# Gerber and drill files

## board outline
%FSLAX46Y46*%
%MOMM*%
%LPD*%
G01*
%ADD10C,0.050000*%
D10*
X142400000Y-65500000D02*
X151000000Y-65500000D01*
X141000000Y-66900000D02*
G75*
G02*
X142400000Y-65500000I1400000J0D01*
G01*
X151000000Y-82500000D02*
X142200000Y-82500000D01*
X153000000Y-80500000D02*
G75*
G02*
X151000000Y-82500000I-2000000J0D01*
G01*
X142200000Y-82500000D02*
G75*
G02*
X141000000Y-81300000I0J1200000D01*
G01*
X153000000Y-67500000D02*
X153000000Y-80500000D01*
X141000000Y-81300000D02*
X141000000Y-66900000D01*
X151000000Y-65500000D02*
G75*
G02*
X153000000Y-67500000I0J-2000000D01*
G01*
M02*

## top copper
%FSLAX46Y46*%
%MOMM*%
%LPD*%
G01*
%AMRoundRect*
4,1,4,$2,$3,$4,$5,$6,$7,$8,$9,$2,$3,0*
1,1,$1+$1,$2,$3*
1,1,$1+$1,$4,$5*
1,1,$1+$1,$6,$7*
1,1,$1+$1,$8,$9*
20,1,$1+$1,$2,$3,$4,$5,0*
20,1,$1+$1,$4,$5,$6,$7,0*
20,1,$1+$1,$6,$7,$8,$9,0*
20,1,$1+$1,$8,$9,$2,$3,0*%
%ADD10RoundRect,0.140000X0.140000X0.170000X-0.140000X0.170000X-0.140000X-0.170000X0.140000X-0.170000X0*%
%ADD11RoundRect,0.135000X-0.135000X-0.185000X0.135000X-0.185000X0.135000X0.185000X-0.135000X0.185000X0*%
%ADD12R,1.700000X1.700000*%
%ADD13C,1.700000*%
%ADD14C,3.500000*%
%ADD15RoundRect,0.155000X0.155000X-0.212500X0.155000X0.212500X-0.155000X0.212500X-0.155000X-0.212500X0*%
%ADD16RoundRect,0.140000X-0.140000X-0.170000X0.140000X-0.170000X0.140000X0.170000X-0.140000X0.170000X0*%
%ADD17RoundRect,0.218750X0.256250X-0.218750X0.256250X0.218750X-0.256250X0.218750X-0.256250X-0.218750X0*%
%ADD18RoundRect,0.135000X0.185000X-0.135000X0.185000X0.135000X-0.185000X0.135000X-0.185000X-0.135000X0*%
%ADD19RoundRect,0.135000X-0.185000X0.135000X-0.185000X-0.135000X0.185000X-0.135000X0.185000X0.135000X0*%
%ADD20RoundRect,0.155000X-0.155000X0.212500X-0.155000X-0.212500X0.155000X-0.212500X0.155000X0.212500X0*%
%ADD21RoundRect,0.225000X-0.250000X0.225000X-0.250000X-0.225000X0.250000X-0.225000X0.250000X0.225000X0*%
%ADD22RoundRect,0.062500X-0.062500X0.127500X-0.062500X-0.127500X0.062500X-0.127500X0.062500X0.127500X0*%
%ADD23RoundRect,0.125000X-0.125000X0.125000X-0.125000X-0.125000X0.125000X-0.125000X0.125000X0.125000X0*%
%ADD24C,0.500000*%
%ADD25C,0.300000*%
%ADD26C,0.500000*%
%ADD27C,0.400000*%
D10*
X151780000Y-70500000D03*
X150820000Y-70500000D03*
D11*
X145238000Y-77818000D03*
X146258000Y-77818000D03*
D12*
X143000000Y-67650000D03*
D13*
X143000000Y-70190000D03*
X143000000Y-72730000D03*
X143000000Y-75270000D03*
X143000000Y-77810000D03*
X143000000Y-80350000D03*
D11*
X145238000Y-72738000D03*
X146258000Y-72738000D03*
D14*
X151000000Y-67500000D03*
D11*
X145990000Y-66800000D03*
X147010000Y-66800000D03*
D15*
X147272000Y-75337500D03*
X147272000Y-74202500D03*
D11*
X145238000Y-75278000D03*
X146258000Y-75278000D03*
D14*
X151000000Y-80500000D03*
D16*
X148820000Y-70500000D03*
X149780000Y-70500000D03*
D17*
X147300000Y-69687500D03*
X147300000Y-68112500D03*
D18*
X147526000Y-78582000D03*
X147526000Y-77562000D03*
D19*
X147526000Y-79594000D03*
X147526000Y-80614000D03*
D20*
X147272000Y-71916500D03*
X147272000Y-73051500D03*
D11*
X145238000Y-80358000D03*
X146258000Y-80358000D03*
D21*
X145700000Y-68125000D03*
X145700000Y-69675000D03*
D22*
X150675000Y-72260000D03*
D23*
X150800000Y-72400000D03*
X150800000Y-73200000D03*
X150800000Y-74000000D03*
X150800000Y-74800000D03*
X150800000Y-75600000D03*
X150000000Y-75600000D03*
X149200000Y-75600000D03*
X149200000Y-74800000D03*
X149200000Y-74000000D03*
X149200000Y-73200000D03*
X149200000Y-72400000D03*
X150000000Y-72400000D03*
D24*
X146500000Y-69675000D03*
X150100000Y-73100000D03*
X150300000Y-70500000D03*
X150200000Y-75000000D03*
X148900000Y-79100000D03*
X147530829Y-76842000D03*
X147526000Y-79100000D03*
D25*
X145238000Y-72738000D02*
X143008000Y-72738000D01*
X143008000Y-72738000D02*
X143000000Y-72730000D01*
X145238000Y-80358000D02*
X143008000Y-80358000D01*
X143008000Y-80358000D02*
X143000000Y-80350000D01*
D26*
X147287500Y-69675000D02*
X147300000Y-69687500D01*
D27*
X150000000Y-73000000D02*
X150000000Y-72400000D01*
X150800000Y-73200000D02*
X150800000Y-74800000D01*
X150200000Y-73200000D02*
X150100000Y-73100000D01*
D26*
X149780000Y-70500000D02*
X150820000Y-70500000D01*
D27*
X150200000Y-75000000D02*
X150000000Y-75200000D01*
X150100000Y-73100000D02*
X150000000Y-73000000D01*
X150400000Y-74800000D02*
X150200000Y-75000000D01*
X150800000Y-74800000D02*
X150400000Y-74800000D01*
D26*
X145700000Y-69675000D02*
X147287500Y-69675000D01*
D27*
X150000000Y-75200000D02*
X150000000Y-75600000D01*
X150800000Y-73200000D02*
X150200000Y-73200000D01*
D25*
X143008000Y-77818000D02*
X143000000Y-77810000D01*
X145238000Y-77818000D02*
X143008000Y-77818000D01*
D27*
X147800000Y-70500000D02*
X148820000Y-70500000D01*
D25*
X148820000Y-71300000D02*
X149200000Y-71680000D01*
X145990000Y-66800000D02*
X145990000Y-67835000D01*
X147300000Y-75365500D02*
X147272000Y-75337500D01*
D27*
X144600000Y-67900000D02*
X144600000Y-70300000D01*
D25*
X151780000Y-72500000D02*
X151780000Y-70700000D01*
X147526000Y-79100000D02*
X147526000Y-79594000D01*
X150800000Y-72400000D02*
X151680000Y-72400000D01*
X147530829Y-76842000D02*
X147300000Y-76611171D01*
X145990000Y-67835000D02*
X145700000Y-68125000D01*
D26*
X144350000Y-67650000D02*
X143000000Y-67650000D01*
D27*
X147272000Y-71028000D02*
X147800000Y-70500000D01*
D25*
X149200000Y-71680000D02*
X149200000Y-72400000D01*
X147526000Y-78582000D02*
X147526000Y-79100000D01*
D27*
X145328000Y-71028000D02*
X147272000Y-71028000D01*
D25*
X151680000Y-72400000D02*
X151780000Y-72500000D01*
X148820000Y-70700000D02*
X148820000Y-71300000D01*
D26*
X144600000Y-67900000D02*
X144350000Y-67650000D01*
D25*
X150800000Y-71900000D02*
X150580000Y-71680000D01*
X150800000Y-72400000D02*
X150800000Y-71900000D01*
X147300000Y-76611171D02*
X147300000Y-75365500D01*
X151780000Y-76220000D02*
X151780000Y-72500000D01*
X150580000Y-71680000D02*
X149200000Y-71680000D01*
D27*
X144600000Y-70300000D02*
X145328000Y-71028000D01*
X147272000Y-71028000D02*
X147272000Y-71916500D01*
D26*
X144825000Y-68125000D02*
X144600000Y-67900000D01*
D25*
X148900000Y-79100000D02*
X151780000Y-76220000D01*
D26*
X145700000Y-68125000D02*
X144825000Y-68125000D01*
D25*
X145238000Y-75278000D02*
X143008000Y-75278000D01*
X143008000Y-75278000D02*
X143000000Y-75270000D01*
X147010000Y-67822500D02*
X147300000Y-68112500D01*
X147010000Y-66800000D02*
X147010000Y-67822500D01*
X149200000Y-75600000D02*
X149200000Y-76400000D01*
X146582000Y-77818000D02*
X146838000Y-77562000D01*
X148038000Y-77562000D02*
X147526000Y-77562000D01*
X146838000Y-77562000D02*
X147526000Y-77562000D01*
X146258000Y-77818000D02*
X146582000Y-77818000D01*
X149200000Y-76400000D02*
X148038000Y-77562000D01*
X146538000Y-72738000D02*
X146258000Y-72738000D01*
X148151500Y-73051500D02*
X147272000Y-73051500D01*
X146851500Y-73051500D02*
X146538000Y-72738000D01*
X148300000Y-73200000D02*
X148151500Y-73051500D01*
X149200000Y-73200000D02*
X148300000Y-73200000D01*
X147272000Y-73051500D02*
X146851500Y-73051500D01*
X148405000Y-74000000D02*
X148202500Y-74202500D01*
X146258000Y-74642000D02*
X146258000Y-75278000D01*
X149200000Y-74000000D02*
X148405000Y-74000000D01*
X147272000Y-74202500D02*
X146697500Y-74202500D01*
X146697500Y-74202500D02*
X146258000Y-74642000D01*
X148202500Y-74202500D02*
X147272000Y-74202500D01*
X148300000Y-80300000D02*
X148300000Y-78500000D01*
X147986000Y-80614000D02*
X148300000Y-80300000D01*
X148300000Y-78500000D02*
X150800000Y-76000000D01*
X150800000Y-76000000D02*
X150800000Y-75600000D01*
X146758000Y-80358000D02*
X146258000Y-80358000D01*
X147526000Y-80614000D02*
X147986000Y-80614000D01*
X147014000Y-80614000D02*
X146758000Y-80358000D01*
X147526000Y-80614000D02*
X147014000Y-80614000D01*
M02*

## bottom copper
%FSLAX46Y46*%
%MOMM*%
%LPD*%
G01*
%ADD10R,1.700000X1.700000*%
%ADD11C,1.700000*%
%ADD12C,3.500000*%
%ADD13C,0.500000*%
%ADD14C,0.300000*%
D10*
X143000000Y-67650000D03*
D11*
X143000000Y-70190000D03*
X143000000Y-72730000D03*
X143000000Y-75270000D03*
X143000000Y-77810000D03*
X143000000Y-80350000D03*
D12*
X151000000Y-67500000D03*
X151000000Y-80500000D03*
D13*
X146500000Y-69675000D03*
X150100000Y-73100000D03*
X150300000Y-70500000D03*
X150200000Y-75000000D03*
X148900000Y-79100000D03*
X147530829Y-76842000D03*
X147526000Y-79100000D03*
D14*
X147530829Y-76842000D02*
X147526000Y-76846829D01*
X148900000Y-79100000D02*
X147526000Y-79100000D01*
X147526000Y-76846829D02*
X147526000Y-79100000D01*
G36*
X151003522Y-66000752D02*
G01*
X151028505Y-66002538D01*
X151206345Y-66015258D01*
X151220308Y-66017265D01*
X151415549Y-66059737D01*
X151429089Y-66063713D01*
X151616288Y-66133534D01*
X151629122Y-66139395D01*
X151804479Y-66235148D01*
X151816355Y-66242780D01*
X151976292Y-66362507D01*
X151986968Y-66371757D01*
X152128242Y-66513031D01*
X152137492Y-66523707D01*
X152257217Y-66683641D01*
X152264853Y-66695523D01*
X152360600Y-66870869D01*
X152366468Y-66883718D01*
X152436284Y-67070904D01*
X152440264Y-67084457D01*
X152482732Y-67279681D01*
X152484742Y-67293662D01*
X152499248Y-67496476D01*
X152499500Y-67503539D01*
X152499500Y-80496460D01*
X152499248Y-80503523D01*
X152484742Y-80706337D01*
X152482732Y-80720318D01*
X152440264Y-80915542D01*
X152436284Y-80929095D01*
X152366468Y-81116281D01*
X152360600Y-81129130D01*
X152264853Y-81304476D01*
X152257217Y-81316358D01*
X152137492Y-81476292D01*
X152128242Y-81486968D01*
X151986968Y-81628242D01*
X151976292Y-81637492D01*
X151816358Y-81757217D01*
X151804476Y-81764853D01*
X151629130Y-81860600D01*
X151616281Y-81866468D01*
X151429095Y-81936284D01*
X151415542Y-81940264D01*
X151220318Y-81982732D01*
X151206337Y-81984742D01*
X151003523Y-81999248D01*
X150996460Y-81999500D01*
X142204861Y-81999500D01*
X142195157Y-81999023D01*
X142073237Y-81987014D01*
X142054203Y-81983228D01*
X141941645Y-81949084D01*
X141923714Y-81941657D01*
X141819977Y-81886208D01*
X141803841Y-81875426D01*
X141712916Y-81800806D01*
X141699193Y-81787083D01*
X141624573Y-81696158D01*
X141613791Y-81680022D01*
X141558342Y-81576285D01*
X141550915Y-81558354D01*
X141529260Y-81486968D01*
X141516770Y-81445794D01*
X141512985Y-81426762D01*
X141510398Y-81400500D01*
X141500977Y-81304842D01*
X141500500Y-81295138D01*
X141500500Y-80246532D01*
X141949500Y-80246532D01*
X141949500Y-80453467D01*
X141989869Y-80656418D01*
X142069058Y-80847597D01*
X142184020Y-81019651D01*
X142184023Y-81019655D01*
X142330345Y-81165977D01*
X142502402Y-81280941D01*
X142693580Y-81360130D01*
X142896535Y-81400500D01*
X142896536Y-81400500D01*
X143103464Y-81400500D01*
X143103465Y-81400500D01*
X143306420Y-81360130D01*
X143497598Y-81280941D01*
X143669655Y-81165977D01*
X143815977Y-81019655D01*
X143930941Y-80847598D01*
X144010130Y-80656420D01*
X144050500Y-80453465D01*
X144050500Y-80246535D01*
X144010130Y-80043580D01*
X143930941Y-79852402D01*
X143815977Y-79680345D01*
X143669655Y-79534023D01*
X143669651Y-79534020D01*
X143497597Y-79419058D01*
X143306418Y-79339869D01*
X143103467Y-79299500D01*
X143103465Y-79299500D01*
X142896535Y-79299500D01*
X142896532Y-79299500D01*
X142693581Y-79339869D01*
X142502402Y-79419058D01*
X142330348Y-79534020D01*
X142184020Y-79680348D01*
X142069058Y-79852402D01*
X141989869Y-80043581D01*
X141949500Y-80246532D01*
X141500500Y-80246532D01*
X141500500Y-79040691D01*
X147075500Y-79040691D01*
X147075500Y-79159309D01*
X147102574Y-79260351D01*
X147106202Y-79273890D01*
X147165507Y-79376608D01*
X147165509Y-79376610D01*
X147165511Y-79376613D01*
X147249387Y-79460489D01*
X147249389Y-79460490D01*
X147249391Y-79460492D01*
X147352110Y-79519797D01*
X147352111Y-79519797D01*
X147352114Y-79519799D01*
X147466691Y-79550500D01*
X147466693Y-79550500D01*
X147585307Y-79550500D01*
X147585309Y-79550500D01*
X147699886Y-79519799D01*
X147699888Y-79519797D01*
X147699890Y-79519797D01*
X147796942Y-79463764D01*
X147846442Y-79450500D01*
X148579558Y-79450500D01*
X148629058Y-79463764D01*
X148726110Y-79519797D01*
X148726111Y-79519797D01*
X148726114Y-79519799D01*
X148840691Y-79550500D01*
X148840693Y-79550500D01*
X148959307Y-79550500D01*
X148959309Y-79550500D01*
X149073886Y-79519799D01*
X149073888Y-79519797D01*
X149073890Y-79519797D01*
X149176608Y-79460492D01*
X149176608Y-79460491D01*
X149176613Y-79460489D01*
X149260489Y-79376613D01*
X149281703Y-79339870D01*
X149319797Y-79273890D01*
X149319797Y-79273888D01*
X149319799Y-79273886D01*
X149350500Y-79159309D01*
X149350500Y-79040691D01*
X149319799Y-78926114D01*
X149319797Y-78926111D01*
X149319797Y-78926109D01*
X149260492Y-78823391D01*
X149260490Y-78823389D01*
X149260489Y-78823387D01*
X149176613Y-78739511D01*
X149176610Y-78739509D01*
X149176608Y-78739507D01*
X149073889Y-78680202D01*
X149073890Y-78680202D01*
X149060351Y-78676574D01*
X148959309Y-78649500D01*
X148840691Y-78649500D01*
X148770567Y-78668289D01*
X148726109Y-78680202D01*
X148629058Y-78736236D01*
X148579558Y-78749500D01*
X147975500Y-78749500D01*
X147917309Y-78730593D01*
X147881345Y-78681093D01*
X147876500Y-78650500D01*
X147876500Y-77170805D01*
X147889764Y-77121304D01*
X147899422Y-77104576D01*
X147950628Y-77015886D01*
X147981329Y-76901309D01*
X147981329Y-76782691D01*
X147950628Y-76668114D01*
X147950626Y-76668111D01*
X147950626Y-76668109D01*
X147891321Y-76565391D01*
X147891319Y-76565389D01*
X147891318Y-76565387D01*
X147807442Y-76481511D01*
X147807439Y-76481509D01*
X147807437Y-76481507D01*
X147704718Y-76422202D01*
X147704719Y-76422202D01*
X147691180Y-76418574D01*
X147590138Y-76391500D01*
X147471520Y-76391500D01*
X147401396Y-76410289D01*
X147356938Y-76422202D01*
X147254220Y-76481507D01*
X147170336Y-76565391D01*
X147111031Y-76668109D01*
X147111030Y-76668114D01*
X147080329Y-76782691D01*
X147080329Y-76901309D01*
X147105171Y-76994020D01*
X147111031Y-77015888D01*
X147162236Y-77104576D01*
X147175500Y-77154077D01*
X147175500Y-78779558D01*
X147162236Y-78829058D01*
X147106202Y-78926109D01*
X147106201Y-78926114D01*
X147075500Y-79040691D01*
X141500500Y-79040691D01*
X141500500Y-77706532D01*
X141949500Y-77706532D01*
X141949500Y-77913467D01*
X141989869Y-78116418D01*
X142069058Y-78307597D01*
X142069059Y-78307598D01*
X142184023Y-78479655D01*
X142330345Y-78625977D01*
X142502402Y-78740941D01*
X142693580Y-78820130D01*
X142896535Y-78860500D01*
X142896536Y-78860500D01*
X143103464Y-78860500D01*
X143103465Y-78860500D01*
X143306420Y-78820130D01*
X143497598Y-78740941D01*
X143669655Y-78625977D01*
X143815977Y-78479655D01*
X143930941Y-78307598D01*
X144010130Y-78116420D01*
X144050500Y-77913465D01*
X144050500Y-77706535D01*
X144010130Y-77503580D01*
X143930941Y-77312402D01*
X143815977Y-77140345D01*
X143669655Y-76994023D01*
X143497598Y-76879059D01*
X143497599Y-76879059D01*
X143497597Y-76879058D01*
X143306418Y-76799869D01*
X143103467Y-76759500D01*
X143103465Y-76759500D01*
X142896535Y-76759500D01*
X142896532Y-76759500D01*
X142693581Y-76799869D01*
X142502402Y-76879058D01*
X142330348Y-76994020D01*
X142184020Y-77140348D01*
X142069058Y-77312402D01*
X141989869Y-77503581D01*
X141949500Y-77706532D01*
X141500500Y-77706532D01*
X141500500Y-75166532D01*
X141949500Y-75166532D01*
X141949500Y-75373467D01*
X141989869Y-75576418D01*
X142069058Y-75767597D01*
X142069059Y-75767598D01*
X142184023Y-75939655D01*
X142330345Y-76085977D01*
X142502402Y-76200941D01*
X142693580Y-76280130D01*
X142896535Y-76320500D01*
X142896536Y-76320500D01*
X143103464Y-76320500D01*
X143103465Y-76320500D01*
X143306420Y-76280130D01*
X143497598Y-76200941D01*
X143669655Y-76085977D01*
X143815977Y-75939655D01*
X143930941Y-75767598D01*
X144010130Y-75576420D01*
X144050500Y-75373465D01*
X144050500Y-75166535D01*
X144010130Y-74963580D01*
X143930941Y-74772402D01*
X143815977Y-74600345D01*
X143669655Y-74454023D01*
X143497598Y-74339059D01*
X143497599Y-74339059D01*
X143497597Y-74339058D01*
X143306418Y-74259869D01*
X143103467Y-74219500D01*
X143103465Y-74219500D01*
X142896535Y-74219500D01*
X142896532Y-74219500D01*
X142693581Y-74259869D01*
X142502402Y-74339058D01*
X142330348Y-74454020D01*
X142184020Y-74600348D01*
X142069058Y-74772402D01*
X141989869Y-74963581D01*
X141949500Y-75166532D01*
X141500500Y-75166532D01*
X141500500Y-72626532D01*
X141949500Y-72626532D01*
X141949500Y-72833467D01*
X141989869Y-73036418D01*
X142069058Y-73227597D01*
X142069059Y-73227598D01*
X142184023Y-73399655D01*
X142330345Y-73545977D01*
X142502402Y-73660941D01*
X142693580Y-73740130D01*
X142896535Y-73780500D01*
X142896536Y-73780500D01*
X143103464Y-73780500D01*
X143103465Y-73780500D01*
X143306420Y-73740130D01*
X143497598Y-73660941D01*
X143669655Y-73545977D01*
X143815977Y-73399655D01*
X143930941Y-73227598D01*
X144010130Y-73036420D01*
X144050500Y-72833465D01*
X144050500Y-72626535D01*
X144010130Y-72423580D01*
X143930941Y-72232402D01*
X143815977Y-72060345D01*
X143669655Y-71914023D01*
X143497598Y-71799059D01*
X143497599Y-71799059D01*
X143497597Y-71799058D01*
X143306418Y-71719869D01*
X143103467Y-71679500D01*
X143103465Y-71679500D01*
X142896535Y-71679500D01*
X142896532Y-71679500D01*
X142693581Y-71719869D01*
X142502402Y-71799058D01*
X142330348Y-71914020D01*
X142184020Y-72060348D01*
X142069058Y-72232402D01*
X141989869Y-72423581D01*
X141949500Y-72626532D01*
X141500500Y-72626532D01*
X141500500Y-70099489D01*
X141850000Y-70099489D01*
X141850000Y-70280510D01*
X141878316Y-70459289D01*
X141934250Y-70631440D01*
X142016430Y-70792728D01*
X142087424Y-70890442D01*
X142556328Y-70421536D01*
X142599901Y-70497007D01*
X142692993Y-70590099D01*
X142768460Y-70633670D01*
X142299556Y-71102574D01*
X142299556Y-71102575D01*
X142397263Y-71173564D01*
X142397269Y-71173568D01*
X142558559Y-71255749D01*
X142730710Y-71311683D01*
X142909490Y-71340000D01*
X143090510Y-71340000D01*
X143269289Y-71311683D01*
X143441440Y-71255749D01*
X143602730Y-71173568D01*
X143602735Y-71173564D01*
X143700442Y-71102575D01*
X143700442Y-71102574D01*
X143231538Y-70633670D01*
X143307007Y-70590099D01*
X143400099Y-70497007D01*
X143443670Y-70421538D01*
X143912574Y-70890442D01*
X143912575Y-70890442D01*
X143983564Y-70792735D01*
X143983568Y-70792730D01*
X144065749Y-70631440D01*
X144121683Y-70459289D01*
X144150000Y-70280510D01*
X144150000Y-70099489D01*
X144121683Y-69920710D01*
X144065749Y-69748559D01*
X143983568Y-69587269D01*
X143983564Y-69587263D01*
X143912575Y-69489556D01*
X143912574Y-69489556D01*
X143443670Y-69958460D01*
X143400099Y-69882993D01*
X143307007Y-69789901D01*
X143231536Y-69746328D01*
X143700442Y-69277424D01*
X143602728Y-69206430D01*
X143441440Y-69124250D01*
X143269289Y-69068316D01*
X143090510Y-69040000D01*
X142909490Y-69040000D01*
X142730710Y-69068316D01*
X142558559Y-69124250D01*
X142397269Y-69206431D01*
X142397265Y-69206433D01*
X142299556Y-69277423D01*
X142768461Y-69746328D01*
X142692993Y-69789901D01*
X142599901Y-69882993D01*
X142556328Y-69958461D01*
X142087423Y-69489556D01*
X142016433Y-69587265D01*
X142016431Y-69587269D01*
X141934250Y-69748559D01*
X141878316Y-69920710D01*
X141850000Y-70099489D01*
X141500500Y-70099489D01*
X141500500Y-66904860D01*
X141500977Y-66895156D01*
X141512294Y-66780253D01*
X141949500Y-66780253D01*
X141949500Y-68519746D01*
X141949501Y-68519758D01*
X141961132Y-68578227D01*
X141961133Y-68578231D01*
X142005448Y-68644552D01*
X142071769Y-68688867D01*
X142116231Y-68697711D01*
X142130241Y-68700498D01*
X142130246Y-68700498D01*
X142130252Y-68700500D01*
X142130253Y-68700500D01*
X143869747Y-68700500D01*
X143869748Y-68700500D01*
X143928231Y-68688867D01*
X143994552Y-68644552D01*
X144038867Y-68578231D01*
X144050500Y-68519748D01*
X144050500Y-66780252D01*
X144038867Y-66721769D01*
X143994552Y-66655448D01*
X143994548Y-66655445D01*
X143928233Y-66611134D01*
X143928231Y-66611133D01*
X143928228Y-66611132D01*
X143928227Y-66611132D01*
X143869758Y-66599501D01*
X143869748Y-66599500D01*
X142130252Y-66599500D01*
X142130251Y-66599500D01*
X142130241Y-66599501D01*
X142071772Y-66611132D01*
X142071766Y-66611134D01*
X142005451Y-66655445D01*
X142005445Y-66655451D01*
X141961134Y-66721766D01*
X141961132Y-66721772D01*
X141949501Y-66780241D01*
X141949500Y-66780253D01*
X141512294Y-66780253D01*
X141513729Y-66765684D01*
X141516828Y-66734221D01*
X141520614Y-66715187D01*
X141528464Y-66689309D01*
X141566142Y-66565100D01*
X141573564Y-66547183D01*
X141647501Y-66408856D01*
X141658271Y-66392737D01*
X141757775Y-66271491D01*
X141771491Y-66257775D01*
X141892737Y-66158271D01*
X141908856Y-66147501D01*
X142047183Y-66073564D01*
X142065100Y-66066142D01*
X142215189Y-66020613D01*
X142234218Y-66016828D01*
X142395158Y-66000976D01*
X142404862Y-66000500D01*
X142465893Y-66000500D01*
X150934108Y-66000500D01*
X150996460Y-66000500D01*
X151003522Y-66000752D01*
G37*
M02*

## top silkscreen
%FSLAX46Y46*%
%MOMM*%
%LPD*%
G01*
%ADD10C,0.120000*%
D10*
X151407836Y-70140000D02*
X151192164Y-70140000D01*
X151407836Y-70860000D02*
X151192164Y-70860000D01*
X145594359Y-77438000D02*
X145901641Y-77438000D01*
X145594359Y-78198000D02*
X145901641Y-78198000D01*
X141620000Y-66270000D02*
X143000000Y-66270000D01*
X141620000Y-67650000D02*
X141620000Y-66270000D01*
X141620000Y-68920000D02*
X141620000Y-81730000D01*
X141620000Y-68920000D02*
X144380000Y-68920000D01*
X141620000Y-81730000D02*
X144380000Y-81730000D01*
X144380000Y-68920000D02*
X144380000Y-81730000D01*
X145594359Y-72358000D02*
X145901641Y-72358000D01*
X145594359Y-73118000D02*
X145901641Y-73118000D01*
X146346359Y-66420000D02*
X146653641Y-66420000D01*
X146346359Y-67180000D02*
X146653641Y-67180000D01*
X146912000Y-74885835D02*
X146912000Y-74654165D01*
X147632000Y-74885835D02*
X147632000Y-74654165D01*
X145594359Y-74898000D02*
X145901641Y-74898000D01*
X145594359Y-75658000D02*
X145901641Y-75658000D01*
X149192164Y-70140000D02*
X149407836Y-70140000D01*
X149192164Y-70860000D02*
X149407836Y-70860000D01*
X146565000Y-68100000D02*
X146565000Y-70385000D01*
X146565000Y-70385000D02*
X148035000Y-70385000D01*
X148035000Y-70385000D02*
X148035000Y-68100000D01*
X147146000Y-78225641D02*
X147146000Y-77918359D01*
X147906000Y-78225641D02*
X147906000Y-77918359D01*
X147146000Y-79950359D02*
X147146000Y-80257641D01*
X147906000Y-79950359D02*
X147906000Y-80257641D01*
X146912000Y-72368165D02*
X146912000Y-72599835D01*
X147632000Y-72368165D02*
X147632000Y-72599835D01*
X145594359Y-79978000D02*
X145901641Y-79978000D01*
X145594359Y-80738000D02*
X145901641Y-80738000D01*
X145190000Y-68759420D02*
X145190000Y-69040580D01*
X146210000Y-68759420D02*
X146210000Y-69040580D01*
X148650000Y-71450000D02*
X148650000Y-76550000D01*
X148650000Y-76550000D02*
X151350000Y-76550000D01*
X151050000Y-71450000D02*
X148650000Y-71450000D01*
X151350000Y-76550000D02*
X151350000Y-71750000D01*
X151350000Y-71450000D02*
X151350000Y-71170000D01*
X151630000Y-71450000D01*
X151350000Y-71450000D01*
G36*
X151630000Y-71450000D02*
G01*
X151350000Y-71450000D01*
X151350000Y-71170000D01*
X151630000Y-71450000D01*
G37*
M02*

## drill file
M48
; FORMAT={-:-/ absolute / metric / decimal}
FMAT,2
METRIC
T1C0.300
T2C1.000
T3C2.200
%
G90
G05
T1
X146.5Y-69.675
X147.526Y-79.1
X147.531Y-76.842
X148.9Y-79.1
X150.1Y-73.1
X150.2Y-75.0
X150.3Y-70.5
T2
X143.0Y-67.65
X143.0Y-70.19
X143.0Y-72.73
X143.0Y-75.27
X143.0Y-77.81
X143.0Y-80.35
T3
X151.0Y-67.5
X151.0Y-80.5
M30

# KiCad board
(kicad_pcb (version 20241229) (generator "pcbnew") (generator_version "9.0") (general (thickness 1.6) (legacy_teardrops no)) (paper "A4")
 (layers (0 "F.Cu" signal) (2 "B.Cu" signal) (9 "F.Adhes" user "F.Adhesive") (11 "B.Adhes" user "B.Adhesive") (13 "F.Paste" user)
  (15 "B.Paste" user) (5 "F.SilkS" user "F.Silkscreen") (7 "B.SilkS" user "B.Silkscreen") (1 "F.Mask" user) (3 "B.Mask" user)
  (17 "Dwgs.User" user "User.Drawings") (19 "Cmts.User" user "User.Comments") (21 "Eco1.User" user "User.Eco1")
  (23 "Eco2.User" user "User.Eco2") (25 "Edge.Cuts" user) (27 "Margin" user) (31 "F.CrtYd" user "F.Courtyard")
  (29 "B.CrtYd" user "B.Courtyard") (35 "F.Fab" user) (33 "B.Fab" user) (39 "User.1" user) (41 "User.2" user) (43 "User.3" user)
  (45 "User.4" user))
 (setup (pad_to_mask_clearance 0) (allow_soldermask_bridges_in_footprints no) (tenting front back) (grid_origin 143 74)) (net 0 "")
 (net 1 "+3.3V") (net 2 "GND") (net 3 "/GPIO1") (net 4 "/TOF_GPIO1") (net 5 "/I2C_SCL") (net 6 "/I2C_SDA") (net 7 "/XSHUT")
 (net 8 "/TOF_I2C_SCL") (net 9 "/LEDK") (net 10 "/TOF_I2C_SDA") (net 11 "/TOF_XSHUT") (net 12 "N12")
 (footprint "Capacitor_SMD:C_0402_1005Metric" (layer "F.Cu") (at 151.3 70.5 180)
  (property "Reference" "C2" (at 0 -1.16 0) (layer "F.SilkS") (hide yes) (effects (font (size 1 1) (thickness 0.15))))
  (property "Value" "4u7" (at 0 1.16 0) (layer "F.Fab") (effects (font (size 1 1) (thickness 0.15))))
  (fp_line (start -0.107836 0.36) (end 0.107836 0.36) (stroke (width 0.12) (type solid)) (layer "F.SilkS"))
  (fp_line (start -0.107836 -0.36) (end 0.107836 -0.36) (stroke (width 0.12) (type solid)) (layer "F.SilkS"))
  (pad "1" smd roundrect (at -0.48 0 180) (size 0.56 0.62) (layers "F.Cu" "F.Mask" "F.Paste") (roundrect_rratio 0.25) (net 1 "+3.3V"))
  (pad "2" smd roundrect (at 0.48 0 180) (size 0.56 0.62) (layers "F.Cu" "F.Mask" "F.Paste") (roundrect_rratio 0.25) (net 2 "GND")))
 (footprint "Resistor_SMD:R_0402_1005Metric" (layer "F.Cu") (at 145.748 77.818)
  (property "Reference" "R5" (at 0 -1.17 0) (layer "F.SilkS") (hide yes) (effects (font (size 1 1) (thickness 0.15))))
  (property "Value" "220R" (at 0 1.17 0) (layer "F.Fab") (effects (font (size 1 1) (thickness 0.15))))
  (fp_line (start -0.153641 -0.38) (end 0.153641 -0.38) (stroke (width 0.12) (type solid)) (layer "F.SilkS"))
  (fp_line (start -0.153641 0.38) (end 0.153641 0.38) (stroke (width 0.12) (type solid)) (layer "F.SilkS"))
  (pad "1" smd roundrect (at -0.51 0) (size 0.54 0.64) (layers "F.Cu" "F.Mask" "F.Paste") (roundrect_rratio 0.25) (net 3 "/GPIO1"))
  (pad "2" smd roundrect (at 0.51 0) (size 0.54 0.64) (layers "F.Cu" "F.Mask" "F.Paste") (roundrect_rratio 0.25) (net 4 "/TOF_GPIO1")))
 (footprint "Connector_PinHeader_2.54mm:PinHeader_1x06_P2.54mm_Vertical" (layer "F.Cu") (at 143 67.65)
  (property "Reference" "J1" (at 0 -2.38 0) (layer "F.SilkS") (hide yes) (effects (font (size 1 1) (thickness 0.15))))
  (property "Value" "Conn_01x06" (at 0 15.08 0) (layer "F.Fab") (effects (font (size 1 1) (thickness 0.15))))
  (fp_line (start -1.38 -1.38) (end 0 -1.38) (stroke (width 0.12) (type solid)) (layer "F.SilkS"))
  (fp_line (start -1.38 0) (end -1.38 -1.38) (stroke (width 0.12) (type solid)) (layer "F.SilkS"))
  (fp_line (start -1.38 1.27) (end -1.38 14.08) (stroke (width 0.12) (type solid)) (layer "F.SilkS"))
  (fp_line (start -1.38 1.27) (end 1.38 1.27) (stroke (width 0.12) (type solid)) (layer "F.SilkS"))
  (fp_line (start -1.38 14.08) (end 1.38 14.08) (stroke (width 0.12) (type solid)) (layer "F.SilkS"))
  (fp_line (start 1.38 1.27) (end 1.38 14.08) (stroke (width 0.12) (type solid)) (layer "F.SilkS"))
  (pad "1" thru_hole rect (at 0 0) (size 1.7 1.7) (drill 1) (layers "*.Cu" "*.Mask") (remove_unused_layers no) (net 1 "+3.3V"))
  (pad "2" thru_hole circle (at 0 2.54) (size 1.7 1.7) (drill 1) (layers "*.Cu" "*.Mask") (remove_unused_layers no) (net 2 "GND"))
  (pad "3" thru_hole circle (at 0 5.08) (size 1.7 1.7) (drill 1) (layers "*.Cu" "*.Mask") (remove_unused_layers no) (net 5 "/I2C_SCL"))
  (pad "4" thru_hole circle (at 0 7.62) (size 1.7 1.7) (drill 1) (layers "*.Cu" "*.Mask") (remove_unused_layers no) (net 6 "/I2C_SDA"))
  (pad "5" thru_hole circle (at 0 10.16) (size 1.7 1.7) (drill 1) (layers "*.Cu" "*.Mask") (remove_unused_layers no) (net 3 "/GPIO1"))
  (pad "6" thru_hole circle (at 0 12.7) (size 1.7 1.7) (drill 1) (layers "*.Cu" "*.Mask") (remove_unused_layers no) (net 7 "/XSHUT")))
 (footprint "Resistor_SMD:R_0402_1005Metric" (layer "F.Cu") (at 145.748 72.738)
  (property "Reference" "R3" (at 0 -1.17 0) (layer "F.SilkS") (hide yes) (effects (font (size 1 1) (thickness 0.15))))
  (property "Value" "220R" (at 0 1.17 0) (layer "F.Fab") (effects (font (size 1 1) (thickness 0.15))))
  (fp_line (start -0.153641 -0.38) (end 0.153641 -0.38) (stroke (width 0.12) (type solid)) (layer "F.SilkS"))
  (fp_line (start -0.153641 0.38) (end 0.153641 0.38) (stroke (width 0.12) (type solid)) (layer "F.SilkS"))
  (pad "1" smd roundrect (at -0.51 0) (size 0.54 0.64) (layers "F.Cu" "F.Mask" "F.Paste") (roundrect_rratio 0.25) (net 5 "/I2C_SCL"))
  (pad "2" smd roundrect (at 0.51 0) (size 0.54 0.64) (layers "F.Cu" "F.Mask" "F.Paste") (roundrect_rratio 0.25) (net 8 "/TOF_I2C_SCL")))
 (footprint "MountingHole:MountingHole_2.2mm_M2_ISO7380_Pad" (layer "F.Cu") (at 151 67.5)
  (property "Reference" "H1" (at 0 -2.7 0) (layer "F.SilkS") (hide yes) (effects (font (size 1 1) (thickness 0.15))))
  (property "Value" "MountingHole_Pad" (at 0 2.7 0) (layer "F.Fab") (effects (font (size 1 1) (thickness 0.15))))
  (pad "1" thru_hole circle (at 0 0) (size 3.5 3.5) (drill 2.2) (layers "*.Cu" "*.Mask") (remove_unused_layers no) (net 2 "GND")
   (zone_connect 2)))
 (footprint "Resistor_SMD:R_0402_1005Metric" (layer "F.Cu") (at 146.5 66.8)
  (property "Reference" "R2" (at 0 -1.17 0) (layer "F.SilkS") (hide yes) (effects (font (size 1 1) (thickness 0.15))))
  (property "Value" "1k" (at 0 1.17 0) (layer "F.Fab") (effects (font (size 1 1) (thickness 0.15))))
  (fp_line (start -0.153641 -0.38) (end 0.153641 -0.38) (stroke (width 0.12) (type solid)) (layer "F.SilkS"))
  (fp_line (start -0.153641 0.38) (end 0.153641 0.38) (stroke (width 0.12) (type solid)) (layer "F.SilkS"))
  (pad "1" smd roundrect (at -0.51 0) (size 0.54 0.64) (layers "F.Cu" "F.Mask" "F.Paste") (roundrect_rratio 0.25) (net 1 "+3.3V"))
  (pad "2" smd roundrect (at 0.51 0) (size 0.54 0.64) (layers "F.Cu" "F.Mask" "F.Paste") (roundrect_rratio 0.25) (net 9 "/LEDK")))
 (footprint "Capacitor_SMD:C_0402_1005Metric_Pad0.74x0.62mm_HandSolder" (layer "F.Cu") (at 147.272 74.77 90)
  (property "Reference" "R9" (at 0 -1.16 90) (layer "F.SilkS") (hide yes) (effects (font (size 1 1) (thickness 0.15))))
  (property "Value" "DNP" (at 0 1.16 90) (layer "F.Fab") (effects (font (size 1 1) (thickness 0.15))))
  (fp_line (start -0.115835 -0.36) (end 0.115835 -0.36) (stroke (width 0.12) (type solid)) (layer "F.SilkS"))
  (fp_line (start -0.115835 0.36) (end 0.115835 0.36) (stroke (width 0.12) (type solid)) (layer "F.SilkS"))
  (pad "1" smd roundrect (at -0.5675 0 90) (size 0.735 0.62) (layers "F.Cu" "F.Mask" "F.Paste") (roundrect_rratio 0.25) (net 1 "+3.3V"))
  (pad "2" smd roundrect (at 0.5675 0 90) (size 0.735 0.62) (layers "F.Cu" "F.Mask" "F.Paste") (roundrect_rratio 0.25)
   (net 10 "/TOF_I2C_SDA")))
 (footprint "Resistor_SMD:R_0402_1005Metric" (layer "F.Cu") (at 145.748 75.278)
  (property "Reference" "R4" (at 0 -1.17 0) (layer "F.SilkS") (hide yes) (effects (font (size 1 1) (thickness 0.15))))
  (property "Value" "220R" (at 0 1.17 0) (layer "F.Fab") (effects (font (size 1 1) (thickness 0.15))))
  (fp_line (start -0.153641 -0.38) (end 0.153641 -0.38) (stroke (width 0.12) (type solid)) (layer "F.SilkS"))
  (fp_line (start -0.153641 0.38) (end 0.153641 0.38) (stroke (width 0.12) (type solid)) (layer "F.SilkS"))
  (pad "1" smd roundrect (at -0.51 0) (size 0.54 0.64) (layers "F.Cu" "F.Mask" "F.Paste") (roundrect_rratio 0.25) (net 6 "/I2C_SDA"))
  (pad "2" smd roundrect (at 0.51 0) (size 0.54 0.64) (layers "F.Cu" "F.Mask" "F.Paste") (roundrect_rratio 0.25) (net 10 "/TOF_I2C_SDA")))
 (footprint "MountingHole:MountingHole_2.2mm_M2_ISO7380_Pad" (layer "F.Cu") (at 151 80.5)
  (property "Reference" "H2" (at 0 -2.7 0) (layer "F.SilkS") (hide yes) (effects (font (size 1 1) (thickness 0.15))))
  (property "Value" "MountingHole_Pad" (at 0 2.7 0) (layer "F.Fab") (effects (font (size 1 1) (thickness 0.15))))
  (pad "1" thru_hole circle (at 0 0) (size 3.5 3.5) (drill 2.2) (layers "*.Cu" "*.Mask") (remove_unused_layers no) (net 2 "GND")
   (zone_connect 2)))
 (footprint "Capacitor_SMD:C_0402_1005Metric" (layer "F.Cu") (at 149.3 70.5)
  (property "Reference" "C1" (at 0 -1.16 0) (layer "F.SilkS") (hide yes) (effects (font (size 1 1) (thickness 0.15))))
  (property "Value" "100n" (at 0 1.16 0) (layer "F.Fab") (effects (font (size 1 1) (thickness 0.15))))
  (fp_line (start -0.107836 -0.36) (end 0.107836 -0.36) (stroke (width 0.12) (type solid)) (layer "F.SilkS"))
  (fp_line (start -0.107836 0.36) (end 0.107836 0.36) (stroke (width 0.12) (type solid)) (layer "F.SilkS"))
  (pad "1" smd roundrect (at -0.48 0) (size 0.56 0.62) (layers "F.Cu" "F.Mask" "F.Paste") (roundrect_rratio 0.25) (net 1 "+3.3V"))
  (pad "2" smd roundrect (at 0.48 0) (size 0.56 0.62) (layers "F.Cu" "F.Mask" "F.Paste") (roundrect_rratio 0.25) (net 2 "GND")))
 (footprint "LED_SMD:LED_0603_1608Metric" (layer "F.Cu") (at 147.3 68.9 90)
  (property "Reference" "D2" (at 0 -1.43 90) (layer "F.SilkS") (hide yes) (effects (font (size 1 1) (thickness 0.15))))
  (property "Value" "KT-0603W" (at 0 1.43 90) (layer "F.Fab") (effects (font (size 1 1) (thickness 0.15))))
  (fp_line (start 0.8 -0.735) (end -1.485 -0.735) (stroke (width 0.12) (type solid)) (layer "F.SilkS"))
  (fp_line (start -1.485 -0.735) (end -1.485 0.735) (stroke (width 0.12) (type solid)) (layer "F.SilkS"))
  (fp_line (start -1.485 0.735) (end 0.8 0.735) (stroke (width 0.12) (type solid)) (layer "F.SilkS"))
  (pad "1" smd roundrect (at -0.7875 0 90) (size 0.875 0.95) (layers "F.Cu" "F.Mask" "F.Paste") (roundrect_rratio 0.25) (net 2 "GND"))
  (pad "2" smd roundrect (at 0.7875 0 90) (size 0.875 0.95) (layers "F.Cu" "F.Mask" "F.Paste") (roundrect_rratio 0.25) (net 9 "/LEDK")))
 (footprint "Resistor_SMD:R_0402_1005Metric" (layer "F.Cu") (at 147.526 78.072 90)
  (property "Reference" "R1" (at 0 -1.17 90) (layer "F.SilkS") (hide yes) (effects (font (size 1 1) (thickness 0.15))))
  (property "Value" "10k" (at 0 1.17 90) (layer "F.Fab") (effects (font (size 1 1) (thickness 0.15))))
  (fp_line (start -0.153641 -0.38) (end 0.153641 -0.38) (stroke (width 0.12) (type solid)) (layer "F.SilkS"))
  (fp_line (start -0.153641 0.38) (end 0.153641 0.38) (stroke (width 0.12) (type solid)) (layer "F.SilkS"))
  (pad "1" smd roundrect (at -0.51 0 90) (size 0.54 0.64) (layers "F.Cu" "F.Mask" "F.Paste") (roundrect_rratio 0.25) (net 1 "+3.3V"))
  (pad "2" smd roundrect (at 0.51 0 90) (size 0.54 0.64) (layers "F.Cu" "F.Mask" "F.Paste") (roundrect_rratio 0.25) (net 4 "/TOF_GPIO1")))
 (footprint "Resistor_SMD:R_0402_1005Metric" (layer "F.Cu") (at 147.526 80.104 -90)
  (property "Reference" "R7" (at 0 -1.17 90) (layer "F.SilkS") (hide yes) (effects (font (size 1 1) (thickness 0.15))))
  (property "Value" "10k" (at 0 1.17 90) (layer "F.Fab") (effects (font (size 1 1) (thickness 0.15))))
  (fp_line (start -0.153641 0.38) (end 0.153641 0.38) (stroke (width 0.12) (type solid)) (layer "F.SilkS"))
  (fp_line (start -0.153641 -0.38) (end 0.153641 -0.38) (stroke (width 0.12) (type solid)) (layer "F.SilkS"))
  (pad "1" smd roundrect (at -0.51 0 270) (size 0.54 0.64) (layers "F.Cu" "F.Mask" "F.Paste") (roundrect_rratio 0.25) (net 1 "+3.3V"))
  (pad "2" smd roundrect (at 0.51 0 270) (size 0.54 0.64) (layers "F.Cu" "F.Mask" "F.Paste") (roundrect_rratio 0.25) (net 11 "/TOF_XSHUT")))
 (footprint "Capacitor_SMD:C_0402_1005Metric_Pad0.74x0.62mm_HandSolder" (layer "F.Cu") (at 147.272 72.484 -90)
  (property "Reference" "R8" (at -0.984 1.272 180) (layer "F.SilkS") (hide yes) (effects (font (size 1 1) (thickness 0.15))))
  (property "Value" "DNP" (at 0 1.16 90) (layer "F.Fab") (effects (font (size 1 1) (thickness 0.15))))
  (fp_line (start -0.115835 0.36) (end 0.115835 0.36) (stroke (width 0.12) (type solid)) (layer "F.SilkS"))
  (fp_line (start -0.115835 -0.36) (end 0.115835 -0.36) (stroke (width 0.12) (type solid)) (layer "F.SilkS"))
  (pad "1" smd roundrect (at -0.5675 0 270) (size 0.735 0.62) (layers "F.Cu" "F.Mask" "F.Paste") (roundrect_rratio 0.25) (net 1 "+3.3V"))
  (pad "2" smd roundrect (at 0.5675 0 270) (size 0.735 0.62) (layers "F.Cu" "F.Mask" "F.Paste") (roundrect_rratio 0.25)
   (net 8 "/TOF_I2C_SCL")))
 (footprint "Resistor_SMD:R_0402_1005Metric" (layer "F.Cu") (at 145.748 80.358)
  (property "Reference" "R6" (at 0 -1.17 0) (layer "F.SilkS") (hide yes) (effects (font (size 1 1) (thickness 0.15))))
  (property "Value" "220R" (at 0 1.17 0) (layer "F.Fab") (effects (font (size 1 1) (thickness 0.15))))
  (fp_line (start -0.153641 -0.38) (end 0.153641 -0.38) (stroke (width 0.12) (type solid)) (layer "F.SilkS"))
  (fp_line (start -0.153641 0.38) (end 0.153641 0.38) (stroke (width 0.12) (type solid)) (layer "F.SilkS"))
  (pad "1" smd roundrect (at -0.51 0) (size 0.54 0.64) (layers "F.Cu" "F.Mask" "F.Paste") (roundrect_rratio 0.25) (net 7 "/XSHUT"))
  (pad "2" smd roundrect (at 0.51 0) (size 0.54 0.64) (layers "F.Cu" "F.Mask" "F.Paste") (roundrect_rratio 0.25) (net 11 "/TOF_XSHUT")))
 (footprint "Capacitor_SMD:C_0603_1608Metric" (layer "F.Cu") (at 145.7 68.9 -90)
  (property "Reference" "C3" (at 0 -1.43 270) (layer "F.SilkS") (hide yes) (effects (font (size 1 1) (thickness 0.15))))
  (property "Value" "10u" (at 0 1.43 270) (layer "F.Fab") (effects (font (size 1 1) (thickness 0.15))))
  (fp_line (start -0.14058 0.51) (end 0.14058 0.51) (stroke (width 0.12) (type solid)) (layer "F.SilkS"))
  (fp_line (start -0.14058 -0.51) (end 0.14058 -0.51) (stroke (width 0.12) (type solid)) (layer "F.SilkS"))
  (pad "1" smd roundrect (at -0.775 0 270) (size 0.9 0.95) (layers "F.Cu" "F.Mask" "F.Paste") (roundrect_rratio 0.25) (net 1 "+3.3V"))
  (pad "2" smd roundrect (at 0.775 0 270) (size 0.9 0.95) (layers "F.Cu" "F.Mask" "F.Paste") (roundrect_rratio 0.25) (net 2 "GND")))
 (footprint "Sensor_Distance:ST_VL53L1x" (layer "F.Cu") (at 150 74 -90)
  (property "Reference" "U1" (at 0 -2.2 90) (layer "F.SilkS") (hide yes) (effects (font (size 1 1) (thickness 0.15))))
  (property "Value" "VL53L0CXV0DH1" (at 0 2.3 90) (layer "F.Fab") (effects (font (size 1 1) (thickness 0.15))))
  (fp_line (start -2.55 1.35) (end 2.55 1.35) (stroke (width 0.12) (type solid)) (layer "F.SilkS"))
  (fp_line (start 2.55 1.35) (end 2.55 -1.35) (stroke (width 0.12) (type solid)) (layer "F.SilkS"))
  (fp_line (start -2.55 -1.05) (end -2.55 1.35) (stroke (width 0.12) (type solid)) (layer "F.SilkS"))
  (fp_line (start 2.55 -1.35) (end -2.25 -1.35) (stroke (width 0.12) (type solid)) (layer "F.SilkS"))
  (fp_poly
   (pts (xy -2.55 -1.35) (xy -2.83 -1.35) (xy -2.55 -1.63) (xy -2.55 -1.35)) (stroke (width 0.12) (type solid)) (fill yes) (layer "F.SilkS"))
  (pad "1" smd roundrect (at -1.74 -0.675 270) (size 0.38 0.25) (layers "F.Cu" "F.Mask" "F.Paste") (roundrect_rratio 0.25) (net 1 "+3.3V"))
  (pad "1" smd roundrect (at -1.6 -0.8 270) (size 0.5 0.5) (layers "F.Cu" "F.Mask" "F.Paste") (roundrect_rratio 0.25) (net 1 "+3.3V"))
  (pad "2" smd roundrect (at -0.8 -0.8 270) (size 0.5 0.5) (layers "F.Cu" "F.Mask" "F.Paste") (roundrect_rratio 0.25) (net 2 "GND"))
  (pad "3" smd roundrect (at 0 -0.8 270) (size 0.5 0.5) (layers "F.Cu" "F.Mask" "F.Paste") (roundrect_rratio 0.25) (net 2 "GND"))
  (pad "4" smd roundrect (at 0.8 -0.8 270) (size 0.5 0.5) (layers "F.Cu" "F.Mask" "F.Paste") (roundrect_rratio 0.25) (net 2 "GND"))
  (pad "5" smd roundrect (at 1.6 -0.8 270) (size 0.5 0.5) (layers "F.Cu" "F.Mask" "F.Paste") (roundrect_rratio 0.25) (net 11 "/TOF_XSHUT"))
  (pad "6" smd roundrect (at 1.6 0 270) (size 0.5 0.5) (layers "F.Cu" "F.Mask" "F.Paste") (roundrect_rratio 0.25) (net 2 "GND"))
  (pad "7" smd roundrect (at 1.6 0.8 270) (size 0.5 0.5) (layers "F.Cu" "F.Mask" "F.Paste") (roundrect_rratio 0.25) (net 4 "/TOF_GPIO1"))
  (pad "8" smd roundrect (at 0.8 0.8 270) (size 0.5 0.5) (layers "F.Cu" "F.Mask" "F.Paste") (roundrect_rratio 0.25) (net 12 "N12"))
  (pad "9" smd roundrect (at 0 0.8 270) (size 0.5 0.5) (layers "F.Cu" "F.Mask" "F.Paste") (roundrect_rratio 0.25) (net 10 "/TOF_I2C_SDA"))
  (pad "10" smd roundrect (at -0.8 0.8 270) (size 0.5 0.5) (layers "F.Cu" "F.Mask" "F.Paste") (roundrect_rratio 0.25) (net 8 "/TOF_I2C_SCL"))
  (pad "11" smd roundrect (at -1.6 0.8 270) (size 0.5 0.5) (layers "F.Cu" "F.Mask" "F.Paste") (roundrect_rratio 0.25) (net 1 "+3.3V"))
  (pad "12" smd roundrect (at -1.6 0 270) (size 0.5 0.5) (layers "F.Cu" "F.Mask" "F.Paste") (roundrect_rratio 0.25) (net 2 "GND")))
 (gr_line (start 142.4 65.5) (end 151 65.5) (stroke (width 0.05) (type default)) (layer "Edge.Cuts"))
 (gr_arc (start 141 66.9) (mid 141.410051 65.910051) (end 142.4 65.5) (stroke (width 0.05) (type default)) (layer "Edge.Cuts"))
 (gr_line (start 151 82.5) (end 142.2 82.5) (stroke (width 0.05) (type default)) (layer "Edge.Cuts"))
 (gr_arc (start 153 80.5) (mid 152.414214 81.914214) (end 151 82.5) (stroke (width 0.05) (type default)) (layer "Edge.Cuts"))
 (gr_arc (start 142.2 82.5) (mid 141.351472 82.148528) (end 141 81.3) (stroke (width 0.05) (type default)) (layer "Edge.Cuts"))
 (gr_line (start 153 67.5) (end 153 80.5) (stroke (width 0.05) (type default)) (layer "Edge.Cuts"))
 (gr_line (start 141 81.3) (end 141 66.9) (stroke (width 0.05) (type default)) (layer "Edge.Cuts"))
 (gr_arc (start 151 65.5) (mid 152.414214 66.085786) (end 153 67.5) (stroke (width 0.05) (type default)) (layer "Edge.Cuts"))
 (segment (start 145.238 72.738) (end 143.008 72.738) (width 0.3) (layer "F.Cu") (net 5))
 (segment (start 143.008 72.738) (end 143 72.73) (width 0.3) (layer "F.Cu") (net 5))
 (segment (start 145.238 80.358) (end 143.008 80.358) (width 0.3) (layer "F.Cu") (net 7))
 (segment (start 143.008 80.358) (end 143 80.35) (width 0.3) (layer "F.Cu") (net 7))
 (segment (start 147.2875 69.675) (end 147.3 69.6875) (width 0.5) (layer "F.Cu") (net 2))
 (segment (start 150 73) (end 150 72.4) (width 0.4) (layer "F.Cu") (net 2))
 (segment (start 150.8 73.2) (end 150.8 74.8) (width 0.4) (layer "F.Cu") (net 2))
 (segment (start 150.2 73.2) (end 150.1 73.1) (width 0.4) (layer "F.Cu") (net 2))
 (segment (start 149.78 70.5) (end 150.82 70.5) (width 0.5) (layer "F.Cu") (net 2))
 (segment (start 150.2 75) (end 150 75.2) (width 0.4) (layer "F.Cu") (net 2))
 (segment (start 150.1 73.1) (end 150 73) (width 0.4) (layer "F.Cu") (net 2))
 (segment (start 150.4 74.8) (end 150.2 75) (width 0.4) (layer "F.Cu") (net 2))
 (segment (start 150.8 74.8) (end 150.4 74.8) (width 0.4) (layer "F.Cu") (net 2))
 (segment (start 145.7 69.675) (end 147.2875 69.675) (width 0.5) (layer "F.Cu") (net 2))
 (segment (start 150 75.2) (end 150 75.6) (width 0.4) (layer "F.Cu") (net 2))
 (segment (start 150.8 73.2) (end 150.2 73.2) (width 0.4) (layer "F.Cu") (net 2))
 (via (at 146.5 69.675) (size 0.5) (drill 0.3) (layers "F.Cu" "B.Cu") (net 2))
 (via (at 150.1 73.1) (size 0.5) (drill 0.3) (layers "F.Cu" "B.Cu") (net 2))
 (via (at 150.3 70.5) (size 0.5) (drill 0.3) (layers "F.Cu" "B.Cu") (free yes) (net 2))
 (via (at 150.2 75) (size 0.5) (drill 0.3) (layers "F.Cu" "B.Cu") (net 2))
 (segment (start 143.008 77.818) (end 143 77.81) (width 0.3) (layer "F.Cu") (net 3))
 (segment (start 145.238 77.818) (end 143.008 77.818) (width 0.3) (layer "F.Cu") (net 3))
 (segment (start 147.8 70.5) (end 148.82 70.5) (width 0.4) (layer "F.Cu") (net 1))
 (segment (start 148.82 71.3) (end 149.2 71.68) (width 0.3) (layer "F.Cu") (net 1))
 (segment (start 145.99 66.8) (end 145.99 67.835) (width 0.3) (layer "F.Cu") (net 1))
 (segment (start 147.3 75.3655) (end 147.272 75.3375) (width 0.3) (layer "F.Cu") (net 1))
 (segment (start 144.6 67.9) (end 144.6 70.3) (width 0.4) (layer "F.Cu") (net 1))
 (segment (start 151.78 72.5) (end 151.78 70.7) (width 0.3) (layer "F.Cu") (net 1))
 (segment (start 147.526 79.1) (end 147.526 79.594) (width 0.3) (layer "F.Cu") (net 1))
 (segment (start 150.8 72.4) (end 151.68 72.4) (width 0.3) (layer "F.Cu") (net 1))
 (segment (start 147.530829 76.842) (end 147.3 76.611171) (width 0.3) (layer "F.Cu") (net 1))
 (segment (start 145.99 67.835) (end 145.7 68.125) (width 0.3) (layer "F.Cu") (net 1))
 (segment (start 144.35 67.65) (end 143 67.65) (width 0.5) (layer "F.Cu") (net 1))
 (segment (start 147.272 71.028) (end 147.8 70.5) (width 0.4) (layer "F.Cu") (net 1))
 (segment (start 149.2 71.68) (end 149.2 72.4) (width 0.3) (layer "F.Cu") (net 1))
 (segment (start 147.526 78.582) (end 147.526 79.1) (width 0.3) (layer "F.Cu") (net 1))
 (segment (start 145.328 71.028) (end 147.272 71.028) (width 0.4) (layer "F.Cu") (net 1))
 (segment (start 151.68 72.4) (end 151.78 72.5) (width 0.3) (layer "F.Cu") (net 1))
 (segment (start 148.82 70.7) (end 148.82 71.3) (width 0.3) (layer "F.Cu") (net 1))
 (segment (start 144.6 67.9) (end 144.35 67.65) (width 0.5) (layer "F.Cu") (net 1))
 (segment (start 150.8 71.9) (end 150.58 71.68) (width 0.3) (layer "F.Cu") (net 1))
 (segment (start 150.8 72.4) (end 150.8 71.9) (width 0.3) (layer "F.Cu") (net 1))
 (segment (start 147.3 76.611171) (end 147.3 75.3655) (width 0.3) (layer "F.Cu") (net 1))
 (segment (start 151.78 76.22) (end 151.78 72.5) (width 0.3) (layer "F.Cu") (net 1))
 (segment (start 150.58 71.68) (end 149.2 71.68) (width 0.3) (layer "F.Cu") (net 1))
 (segment (start 144.6 70.3) (end 145.328 71.028) (width 0.4) (layer "F.Cu") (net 1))
 (segment (start 147.272 71.028) (end 147.272 71.9165) (width 0.4) (layer "F.Cu") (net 1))
 (segment (start 144.825 68.125) (end 144.6 67.9) (width 0.5) (layer "F.Cu") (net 1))
 (segment (start 148.9 79.1) (end 151.78 76.22) (width 0.3) (layer "F.Cu") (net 1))
 (segment (start 145.7 68.125) (end 144.825 68.125) (width 0.5) (layer "F.Cu") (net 1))
 (via (at 148.9 79.1) (size 0.5) (drill 0.3) (layers "F.Cu" "B.Cu") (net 1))
 (via (at 147.530829 76.842) (size 0.5) (drill 0.3) (layers "F.Cu" "B.Cu") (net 1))
 (via (at 147.526 79.1) (size 0.5) (drill 0.3) (layers "F.Cu" "B.Cu") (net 1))
 (segment (start 147.530829 76.842) (end 147.526 76.846829) (width 0.3) (layer "B.Cu") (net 1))
 (segment (start 148.9 79.1) (end 147.526 79.1) (width 0.3) (layer "B.Cu") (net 1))
 (segment (start 147.526 76.846829) (end 147.526 79.1) (width 0.3) (layer "B.Cu") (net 1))
 (segment (start 145.238 75.278) (end 143.008 75.278) (width 0.3) (layer "F.Cu") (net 6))
 (segment (start 143.008 75.278) (end 143 75.27) (width 0.3) (layer "F.Cu") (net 6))
 (segment (start 147.01 67.8225) (end 147.3 68.1125) (width 0.3) (layer "F.Cu") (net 9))
 (segment (start 147.01 66.8) (end 147.01 67.8225) (width 0.3) (layer "F.Cu") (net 9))
 (segment (start 149.2 75.6) (end 149.2 76.4) (width 0.3) (layer "F.Cu") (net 4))
 (segment (start 146.582 77.818) (end 146.838 77.562) (width 0.3) (layer "F.Cu") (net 4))
 (segment (start 148.038 77.562) (end 147.526 77.562) (width 0.3) (layer "F.Cu") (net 4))
 (segment (start 146.838 77.562) (end 147.526 77.562) (width 0.3) (layer "F.Cu") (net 4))
 (segment (start 146.258 77.818) (end 146.582 77.818) (width 0.3) (layer "F.Cu") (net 4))
 (segment (start 149.2 76.4) (end 148.038 77.562) (width 0.3) (layer "F.Cu") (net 4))
 (segment (start 146.538 72.738) (end 146.258 72.738) (width 0.3) (layer "F.Cu") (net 8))
 (segment (start 148.1515 73.0515) (end 147.272 73.0515) (width 0.3) (layer "F.Cu") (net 8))
 (segment (start 146.8515 73.0515) (end 146.538 72.738) (width 0.3) (layer "F.Cu") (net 8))
 (segment (start 148.3 73.2) (end 148.1515 73.0515) (width 0.3) (layer "F.Cu") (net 8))
 (segment (start 149.2 73.2) (end 148.3 73.2) (width 0.3) (layer "F.Cu") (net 8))
 (segment (start 147.272 73.0515) (end 146.8515 73.0515) (width 0.3) (layer "F.Cu") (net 8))
 (segment (start 148.405 74) (end 148.2025 74.2025) (width 0.3) (layer "F.Cu") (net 10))
 (segment (start 146.258 74.642) (end 146.258 75.278) (width 0.3) (layer "F.Cu") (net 10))
 (segment (start 149.2 74) (end 148.405 74) (width 0.3) (layer "F.Cu") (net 10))
 (segment (start 147.272 74.2025) (end 146.6975 74.2025) (width 0.3) (layer "F.Cu") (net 10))
 (segment (start 146.6975 74.2025) (end 146.258 74.642) (width 0.3) (layer "F.Cu") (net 10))
 (segment (start 148.2025 74.2025) (end 147.272 74.2025) (width 0.3) (layer "F.Cu") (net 10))
 (segment (start 148.3 80.3) (end 148.3 78.5) (width 0.3) (layer "F.Cu") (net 11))
 (segment (start 147.986 80.614) (end 148.3 80.3) (width 0.3) (layer "F.Cu") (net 11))
 (segment (start 148.3 78.5) (end 150.8 76) (width 0.3) (layer "F.Cu") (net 11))
 (segment (start 150.8 76) (end 150.8 75.6) (width 0.3) (layer "F.Cu") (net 11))
 (segment (start 146.758 80.358) (end 146.258 80.358) (width 0.3) (layer "F.Cu") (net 11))
 (segment (start 147.526 80.614) (end 147.986 80.614) (width 0.3) (layer "F.Cu") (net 11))
 (segment (start 147.014 80.614) (end 146.758 80.358) (width 0.3) (layer "F.Cu") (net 11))
 (segment (start 147.526 80.614) (end 147.014 80.614) (width 0.3) (layer "F.Cu") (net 11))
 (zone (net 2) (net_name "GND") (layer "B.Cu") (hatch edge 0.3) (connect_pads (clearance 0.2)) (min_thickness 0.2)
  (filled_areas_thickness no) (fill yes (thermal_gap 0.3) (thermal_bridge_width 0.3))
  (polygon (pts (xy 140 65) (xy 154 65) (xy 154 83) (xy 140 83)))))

